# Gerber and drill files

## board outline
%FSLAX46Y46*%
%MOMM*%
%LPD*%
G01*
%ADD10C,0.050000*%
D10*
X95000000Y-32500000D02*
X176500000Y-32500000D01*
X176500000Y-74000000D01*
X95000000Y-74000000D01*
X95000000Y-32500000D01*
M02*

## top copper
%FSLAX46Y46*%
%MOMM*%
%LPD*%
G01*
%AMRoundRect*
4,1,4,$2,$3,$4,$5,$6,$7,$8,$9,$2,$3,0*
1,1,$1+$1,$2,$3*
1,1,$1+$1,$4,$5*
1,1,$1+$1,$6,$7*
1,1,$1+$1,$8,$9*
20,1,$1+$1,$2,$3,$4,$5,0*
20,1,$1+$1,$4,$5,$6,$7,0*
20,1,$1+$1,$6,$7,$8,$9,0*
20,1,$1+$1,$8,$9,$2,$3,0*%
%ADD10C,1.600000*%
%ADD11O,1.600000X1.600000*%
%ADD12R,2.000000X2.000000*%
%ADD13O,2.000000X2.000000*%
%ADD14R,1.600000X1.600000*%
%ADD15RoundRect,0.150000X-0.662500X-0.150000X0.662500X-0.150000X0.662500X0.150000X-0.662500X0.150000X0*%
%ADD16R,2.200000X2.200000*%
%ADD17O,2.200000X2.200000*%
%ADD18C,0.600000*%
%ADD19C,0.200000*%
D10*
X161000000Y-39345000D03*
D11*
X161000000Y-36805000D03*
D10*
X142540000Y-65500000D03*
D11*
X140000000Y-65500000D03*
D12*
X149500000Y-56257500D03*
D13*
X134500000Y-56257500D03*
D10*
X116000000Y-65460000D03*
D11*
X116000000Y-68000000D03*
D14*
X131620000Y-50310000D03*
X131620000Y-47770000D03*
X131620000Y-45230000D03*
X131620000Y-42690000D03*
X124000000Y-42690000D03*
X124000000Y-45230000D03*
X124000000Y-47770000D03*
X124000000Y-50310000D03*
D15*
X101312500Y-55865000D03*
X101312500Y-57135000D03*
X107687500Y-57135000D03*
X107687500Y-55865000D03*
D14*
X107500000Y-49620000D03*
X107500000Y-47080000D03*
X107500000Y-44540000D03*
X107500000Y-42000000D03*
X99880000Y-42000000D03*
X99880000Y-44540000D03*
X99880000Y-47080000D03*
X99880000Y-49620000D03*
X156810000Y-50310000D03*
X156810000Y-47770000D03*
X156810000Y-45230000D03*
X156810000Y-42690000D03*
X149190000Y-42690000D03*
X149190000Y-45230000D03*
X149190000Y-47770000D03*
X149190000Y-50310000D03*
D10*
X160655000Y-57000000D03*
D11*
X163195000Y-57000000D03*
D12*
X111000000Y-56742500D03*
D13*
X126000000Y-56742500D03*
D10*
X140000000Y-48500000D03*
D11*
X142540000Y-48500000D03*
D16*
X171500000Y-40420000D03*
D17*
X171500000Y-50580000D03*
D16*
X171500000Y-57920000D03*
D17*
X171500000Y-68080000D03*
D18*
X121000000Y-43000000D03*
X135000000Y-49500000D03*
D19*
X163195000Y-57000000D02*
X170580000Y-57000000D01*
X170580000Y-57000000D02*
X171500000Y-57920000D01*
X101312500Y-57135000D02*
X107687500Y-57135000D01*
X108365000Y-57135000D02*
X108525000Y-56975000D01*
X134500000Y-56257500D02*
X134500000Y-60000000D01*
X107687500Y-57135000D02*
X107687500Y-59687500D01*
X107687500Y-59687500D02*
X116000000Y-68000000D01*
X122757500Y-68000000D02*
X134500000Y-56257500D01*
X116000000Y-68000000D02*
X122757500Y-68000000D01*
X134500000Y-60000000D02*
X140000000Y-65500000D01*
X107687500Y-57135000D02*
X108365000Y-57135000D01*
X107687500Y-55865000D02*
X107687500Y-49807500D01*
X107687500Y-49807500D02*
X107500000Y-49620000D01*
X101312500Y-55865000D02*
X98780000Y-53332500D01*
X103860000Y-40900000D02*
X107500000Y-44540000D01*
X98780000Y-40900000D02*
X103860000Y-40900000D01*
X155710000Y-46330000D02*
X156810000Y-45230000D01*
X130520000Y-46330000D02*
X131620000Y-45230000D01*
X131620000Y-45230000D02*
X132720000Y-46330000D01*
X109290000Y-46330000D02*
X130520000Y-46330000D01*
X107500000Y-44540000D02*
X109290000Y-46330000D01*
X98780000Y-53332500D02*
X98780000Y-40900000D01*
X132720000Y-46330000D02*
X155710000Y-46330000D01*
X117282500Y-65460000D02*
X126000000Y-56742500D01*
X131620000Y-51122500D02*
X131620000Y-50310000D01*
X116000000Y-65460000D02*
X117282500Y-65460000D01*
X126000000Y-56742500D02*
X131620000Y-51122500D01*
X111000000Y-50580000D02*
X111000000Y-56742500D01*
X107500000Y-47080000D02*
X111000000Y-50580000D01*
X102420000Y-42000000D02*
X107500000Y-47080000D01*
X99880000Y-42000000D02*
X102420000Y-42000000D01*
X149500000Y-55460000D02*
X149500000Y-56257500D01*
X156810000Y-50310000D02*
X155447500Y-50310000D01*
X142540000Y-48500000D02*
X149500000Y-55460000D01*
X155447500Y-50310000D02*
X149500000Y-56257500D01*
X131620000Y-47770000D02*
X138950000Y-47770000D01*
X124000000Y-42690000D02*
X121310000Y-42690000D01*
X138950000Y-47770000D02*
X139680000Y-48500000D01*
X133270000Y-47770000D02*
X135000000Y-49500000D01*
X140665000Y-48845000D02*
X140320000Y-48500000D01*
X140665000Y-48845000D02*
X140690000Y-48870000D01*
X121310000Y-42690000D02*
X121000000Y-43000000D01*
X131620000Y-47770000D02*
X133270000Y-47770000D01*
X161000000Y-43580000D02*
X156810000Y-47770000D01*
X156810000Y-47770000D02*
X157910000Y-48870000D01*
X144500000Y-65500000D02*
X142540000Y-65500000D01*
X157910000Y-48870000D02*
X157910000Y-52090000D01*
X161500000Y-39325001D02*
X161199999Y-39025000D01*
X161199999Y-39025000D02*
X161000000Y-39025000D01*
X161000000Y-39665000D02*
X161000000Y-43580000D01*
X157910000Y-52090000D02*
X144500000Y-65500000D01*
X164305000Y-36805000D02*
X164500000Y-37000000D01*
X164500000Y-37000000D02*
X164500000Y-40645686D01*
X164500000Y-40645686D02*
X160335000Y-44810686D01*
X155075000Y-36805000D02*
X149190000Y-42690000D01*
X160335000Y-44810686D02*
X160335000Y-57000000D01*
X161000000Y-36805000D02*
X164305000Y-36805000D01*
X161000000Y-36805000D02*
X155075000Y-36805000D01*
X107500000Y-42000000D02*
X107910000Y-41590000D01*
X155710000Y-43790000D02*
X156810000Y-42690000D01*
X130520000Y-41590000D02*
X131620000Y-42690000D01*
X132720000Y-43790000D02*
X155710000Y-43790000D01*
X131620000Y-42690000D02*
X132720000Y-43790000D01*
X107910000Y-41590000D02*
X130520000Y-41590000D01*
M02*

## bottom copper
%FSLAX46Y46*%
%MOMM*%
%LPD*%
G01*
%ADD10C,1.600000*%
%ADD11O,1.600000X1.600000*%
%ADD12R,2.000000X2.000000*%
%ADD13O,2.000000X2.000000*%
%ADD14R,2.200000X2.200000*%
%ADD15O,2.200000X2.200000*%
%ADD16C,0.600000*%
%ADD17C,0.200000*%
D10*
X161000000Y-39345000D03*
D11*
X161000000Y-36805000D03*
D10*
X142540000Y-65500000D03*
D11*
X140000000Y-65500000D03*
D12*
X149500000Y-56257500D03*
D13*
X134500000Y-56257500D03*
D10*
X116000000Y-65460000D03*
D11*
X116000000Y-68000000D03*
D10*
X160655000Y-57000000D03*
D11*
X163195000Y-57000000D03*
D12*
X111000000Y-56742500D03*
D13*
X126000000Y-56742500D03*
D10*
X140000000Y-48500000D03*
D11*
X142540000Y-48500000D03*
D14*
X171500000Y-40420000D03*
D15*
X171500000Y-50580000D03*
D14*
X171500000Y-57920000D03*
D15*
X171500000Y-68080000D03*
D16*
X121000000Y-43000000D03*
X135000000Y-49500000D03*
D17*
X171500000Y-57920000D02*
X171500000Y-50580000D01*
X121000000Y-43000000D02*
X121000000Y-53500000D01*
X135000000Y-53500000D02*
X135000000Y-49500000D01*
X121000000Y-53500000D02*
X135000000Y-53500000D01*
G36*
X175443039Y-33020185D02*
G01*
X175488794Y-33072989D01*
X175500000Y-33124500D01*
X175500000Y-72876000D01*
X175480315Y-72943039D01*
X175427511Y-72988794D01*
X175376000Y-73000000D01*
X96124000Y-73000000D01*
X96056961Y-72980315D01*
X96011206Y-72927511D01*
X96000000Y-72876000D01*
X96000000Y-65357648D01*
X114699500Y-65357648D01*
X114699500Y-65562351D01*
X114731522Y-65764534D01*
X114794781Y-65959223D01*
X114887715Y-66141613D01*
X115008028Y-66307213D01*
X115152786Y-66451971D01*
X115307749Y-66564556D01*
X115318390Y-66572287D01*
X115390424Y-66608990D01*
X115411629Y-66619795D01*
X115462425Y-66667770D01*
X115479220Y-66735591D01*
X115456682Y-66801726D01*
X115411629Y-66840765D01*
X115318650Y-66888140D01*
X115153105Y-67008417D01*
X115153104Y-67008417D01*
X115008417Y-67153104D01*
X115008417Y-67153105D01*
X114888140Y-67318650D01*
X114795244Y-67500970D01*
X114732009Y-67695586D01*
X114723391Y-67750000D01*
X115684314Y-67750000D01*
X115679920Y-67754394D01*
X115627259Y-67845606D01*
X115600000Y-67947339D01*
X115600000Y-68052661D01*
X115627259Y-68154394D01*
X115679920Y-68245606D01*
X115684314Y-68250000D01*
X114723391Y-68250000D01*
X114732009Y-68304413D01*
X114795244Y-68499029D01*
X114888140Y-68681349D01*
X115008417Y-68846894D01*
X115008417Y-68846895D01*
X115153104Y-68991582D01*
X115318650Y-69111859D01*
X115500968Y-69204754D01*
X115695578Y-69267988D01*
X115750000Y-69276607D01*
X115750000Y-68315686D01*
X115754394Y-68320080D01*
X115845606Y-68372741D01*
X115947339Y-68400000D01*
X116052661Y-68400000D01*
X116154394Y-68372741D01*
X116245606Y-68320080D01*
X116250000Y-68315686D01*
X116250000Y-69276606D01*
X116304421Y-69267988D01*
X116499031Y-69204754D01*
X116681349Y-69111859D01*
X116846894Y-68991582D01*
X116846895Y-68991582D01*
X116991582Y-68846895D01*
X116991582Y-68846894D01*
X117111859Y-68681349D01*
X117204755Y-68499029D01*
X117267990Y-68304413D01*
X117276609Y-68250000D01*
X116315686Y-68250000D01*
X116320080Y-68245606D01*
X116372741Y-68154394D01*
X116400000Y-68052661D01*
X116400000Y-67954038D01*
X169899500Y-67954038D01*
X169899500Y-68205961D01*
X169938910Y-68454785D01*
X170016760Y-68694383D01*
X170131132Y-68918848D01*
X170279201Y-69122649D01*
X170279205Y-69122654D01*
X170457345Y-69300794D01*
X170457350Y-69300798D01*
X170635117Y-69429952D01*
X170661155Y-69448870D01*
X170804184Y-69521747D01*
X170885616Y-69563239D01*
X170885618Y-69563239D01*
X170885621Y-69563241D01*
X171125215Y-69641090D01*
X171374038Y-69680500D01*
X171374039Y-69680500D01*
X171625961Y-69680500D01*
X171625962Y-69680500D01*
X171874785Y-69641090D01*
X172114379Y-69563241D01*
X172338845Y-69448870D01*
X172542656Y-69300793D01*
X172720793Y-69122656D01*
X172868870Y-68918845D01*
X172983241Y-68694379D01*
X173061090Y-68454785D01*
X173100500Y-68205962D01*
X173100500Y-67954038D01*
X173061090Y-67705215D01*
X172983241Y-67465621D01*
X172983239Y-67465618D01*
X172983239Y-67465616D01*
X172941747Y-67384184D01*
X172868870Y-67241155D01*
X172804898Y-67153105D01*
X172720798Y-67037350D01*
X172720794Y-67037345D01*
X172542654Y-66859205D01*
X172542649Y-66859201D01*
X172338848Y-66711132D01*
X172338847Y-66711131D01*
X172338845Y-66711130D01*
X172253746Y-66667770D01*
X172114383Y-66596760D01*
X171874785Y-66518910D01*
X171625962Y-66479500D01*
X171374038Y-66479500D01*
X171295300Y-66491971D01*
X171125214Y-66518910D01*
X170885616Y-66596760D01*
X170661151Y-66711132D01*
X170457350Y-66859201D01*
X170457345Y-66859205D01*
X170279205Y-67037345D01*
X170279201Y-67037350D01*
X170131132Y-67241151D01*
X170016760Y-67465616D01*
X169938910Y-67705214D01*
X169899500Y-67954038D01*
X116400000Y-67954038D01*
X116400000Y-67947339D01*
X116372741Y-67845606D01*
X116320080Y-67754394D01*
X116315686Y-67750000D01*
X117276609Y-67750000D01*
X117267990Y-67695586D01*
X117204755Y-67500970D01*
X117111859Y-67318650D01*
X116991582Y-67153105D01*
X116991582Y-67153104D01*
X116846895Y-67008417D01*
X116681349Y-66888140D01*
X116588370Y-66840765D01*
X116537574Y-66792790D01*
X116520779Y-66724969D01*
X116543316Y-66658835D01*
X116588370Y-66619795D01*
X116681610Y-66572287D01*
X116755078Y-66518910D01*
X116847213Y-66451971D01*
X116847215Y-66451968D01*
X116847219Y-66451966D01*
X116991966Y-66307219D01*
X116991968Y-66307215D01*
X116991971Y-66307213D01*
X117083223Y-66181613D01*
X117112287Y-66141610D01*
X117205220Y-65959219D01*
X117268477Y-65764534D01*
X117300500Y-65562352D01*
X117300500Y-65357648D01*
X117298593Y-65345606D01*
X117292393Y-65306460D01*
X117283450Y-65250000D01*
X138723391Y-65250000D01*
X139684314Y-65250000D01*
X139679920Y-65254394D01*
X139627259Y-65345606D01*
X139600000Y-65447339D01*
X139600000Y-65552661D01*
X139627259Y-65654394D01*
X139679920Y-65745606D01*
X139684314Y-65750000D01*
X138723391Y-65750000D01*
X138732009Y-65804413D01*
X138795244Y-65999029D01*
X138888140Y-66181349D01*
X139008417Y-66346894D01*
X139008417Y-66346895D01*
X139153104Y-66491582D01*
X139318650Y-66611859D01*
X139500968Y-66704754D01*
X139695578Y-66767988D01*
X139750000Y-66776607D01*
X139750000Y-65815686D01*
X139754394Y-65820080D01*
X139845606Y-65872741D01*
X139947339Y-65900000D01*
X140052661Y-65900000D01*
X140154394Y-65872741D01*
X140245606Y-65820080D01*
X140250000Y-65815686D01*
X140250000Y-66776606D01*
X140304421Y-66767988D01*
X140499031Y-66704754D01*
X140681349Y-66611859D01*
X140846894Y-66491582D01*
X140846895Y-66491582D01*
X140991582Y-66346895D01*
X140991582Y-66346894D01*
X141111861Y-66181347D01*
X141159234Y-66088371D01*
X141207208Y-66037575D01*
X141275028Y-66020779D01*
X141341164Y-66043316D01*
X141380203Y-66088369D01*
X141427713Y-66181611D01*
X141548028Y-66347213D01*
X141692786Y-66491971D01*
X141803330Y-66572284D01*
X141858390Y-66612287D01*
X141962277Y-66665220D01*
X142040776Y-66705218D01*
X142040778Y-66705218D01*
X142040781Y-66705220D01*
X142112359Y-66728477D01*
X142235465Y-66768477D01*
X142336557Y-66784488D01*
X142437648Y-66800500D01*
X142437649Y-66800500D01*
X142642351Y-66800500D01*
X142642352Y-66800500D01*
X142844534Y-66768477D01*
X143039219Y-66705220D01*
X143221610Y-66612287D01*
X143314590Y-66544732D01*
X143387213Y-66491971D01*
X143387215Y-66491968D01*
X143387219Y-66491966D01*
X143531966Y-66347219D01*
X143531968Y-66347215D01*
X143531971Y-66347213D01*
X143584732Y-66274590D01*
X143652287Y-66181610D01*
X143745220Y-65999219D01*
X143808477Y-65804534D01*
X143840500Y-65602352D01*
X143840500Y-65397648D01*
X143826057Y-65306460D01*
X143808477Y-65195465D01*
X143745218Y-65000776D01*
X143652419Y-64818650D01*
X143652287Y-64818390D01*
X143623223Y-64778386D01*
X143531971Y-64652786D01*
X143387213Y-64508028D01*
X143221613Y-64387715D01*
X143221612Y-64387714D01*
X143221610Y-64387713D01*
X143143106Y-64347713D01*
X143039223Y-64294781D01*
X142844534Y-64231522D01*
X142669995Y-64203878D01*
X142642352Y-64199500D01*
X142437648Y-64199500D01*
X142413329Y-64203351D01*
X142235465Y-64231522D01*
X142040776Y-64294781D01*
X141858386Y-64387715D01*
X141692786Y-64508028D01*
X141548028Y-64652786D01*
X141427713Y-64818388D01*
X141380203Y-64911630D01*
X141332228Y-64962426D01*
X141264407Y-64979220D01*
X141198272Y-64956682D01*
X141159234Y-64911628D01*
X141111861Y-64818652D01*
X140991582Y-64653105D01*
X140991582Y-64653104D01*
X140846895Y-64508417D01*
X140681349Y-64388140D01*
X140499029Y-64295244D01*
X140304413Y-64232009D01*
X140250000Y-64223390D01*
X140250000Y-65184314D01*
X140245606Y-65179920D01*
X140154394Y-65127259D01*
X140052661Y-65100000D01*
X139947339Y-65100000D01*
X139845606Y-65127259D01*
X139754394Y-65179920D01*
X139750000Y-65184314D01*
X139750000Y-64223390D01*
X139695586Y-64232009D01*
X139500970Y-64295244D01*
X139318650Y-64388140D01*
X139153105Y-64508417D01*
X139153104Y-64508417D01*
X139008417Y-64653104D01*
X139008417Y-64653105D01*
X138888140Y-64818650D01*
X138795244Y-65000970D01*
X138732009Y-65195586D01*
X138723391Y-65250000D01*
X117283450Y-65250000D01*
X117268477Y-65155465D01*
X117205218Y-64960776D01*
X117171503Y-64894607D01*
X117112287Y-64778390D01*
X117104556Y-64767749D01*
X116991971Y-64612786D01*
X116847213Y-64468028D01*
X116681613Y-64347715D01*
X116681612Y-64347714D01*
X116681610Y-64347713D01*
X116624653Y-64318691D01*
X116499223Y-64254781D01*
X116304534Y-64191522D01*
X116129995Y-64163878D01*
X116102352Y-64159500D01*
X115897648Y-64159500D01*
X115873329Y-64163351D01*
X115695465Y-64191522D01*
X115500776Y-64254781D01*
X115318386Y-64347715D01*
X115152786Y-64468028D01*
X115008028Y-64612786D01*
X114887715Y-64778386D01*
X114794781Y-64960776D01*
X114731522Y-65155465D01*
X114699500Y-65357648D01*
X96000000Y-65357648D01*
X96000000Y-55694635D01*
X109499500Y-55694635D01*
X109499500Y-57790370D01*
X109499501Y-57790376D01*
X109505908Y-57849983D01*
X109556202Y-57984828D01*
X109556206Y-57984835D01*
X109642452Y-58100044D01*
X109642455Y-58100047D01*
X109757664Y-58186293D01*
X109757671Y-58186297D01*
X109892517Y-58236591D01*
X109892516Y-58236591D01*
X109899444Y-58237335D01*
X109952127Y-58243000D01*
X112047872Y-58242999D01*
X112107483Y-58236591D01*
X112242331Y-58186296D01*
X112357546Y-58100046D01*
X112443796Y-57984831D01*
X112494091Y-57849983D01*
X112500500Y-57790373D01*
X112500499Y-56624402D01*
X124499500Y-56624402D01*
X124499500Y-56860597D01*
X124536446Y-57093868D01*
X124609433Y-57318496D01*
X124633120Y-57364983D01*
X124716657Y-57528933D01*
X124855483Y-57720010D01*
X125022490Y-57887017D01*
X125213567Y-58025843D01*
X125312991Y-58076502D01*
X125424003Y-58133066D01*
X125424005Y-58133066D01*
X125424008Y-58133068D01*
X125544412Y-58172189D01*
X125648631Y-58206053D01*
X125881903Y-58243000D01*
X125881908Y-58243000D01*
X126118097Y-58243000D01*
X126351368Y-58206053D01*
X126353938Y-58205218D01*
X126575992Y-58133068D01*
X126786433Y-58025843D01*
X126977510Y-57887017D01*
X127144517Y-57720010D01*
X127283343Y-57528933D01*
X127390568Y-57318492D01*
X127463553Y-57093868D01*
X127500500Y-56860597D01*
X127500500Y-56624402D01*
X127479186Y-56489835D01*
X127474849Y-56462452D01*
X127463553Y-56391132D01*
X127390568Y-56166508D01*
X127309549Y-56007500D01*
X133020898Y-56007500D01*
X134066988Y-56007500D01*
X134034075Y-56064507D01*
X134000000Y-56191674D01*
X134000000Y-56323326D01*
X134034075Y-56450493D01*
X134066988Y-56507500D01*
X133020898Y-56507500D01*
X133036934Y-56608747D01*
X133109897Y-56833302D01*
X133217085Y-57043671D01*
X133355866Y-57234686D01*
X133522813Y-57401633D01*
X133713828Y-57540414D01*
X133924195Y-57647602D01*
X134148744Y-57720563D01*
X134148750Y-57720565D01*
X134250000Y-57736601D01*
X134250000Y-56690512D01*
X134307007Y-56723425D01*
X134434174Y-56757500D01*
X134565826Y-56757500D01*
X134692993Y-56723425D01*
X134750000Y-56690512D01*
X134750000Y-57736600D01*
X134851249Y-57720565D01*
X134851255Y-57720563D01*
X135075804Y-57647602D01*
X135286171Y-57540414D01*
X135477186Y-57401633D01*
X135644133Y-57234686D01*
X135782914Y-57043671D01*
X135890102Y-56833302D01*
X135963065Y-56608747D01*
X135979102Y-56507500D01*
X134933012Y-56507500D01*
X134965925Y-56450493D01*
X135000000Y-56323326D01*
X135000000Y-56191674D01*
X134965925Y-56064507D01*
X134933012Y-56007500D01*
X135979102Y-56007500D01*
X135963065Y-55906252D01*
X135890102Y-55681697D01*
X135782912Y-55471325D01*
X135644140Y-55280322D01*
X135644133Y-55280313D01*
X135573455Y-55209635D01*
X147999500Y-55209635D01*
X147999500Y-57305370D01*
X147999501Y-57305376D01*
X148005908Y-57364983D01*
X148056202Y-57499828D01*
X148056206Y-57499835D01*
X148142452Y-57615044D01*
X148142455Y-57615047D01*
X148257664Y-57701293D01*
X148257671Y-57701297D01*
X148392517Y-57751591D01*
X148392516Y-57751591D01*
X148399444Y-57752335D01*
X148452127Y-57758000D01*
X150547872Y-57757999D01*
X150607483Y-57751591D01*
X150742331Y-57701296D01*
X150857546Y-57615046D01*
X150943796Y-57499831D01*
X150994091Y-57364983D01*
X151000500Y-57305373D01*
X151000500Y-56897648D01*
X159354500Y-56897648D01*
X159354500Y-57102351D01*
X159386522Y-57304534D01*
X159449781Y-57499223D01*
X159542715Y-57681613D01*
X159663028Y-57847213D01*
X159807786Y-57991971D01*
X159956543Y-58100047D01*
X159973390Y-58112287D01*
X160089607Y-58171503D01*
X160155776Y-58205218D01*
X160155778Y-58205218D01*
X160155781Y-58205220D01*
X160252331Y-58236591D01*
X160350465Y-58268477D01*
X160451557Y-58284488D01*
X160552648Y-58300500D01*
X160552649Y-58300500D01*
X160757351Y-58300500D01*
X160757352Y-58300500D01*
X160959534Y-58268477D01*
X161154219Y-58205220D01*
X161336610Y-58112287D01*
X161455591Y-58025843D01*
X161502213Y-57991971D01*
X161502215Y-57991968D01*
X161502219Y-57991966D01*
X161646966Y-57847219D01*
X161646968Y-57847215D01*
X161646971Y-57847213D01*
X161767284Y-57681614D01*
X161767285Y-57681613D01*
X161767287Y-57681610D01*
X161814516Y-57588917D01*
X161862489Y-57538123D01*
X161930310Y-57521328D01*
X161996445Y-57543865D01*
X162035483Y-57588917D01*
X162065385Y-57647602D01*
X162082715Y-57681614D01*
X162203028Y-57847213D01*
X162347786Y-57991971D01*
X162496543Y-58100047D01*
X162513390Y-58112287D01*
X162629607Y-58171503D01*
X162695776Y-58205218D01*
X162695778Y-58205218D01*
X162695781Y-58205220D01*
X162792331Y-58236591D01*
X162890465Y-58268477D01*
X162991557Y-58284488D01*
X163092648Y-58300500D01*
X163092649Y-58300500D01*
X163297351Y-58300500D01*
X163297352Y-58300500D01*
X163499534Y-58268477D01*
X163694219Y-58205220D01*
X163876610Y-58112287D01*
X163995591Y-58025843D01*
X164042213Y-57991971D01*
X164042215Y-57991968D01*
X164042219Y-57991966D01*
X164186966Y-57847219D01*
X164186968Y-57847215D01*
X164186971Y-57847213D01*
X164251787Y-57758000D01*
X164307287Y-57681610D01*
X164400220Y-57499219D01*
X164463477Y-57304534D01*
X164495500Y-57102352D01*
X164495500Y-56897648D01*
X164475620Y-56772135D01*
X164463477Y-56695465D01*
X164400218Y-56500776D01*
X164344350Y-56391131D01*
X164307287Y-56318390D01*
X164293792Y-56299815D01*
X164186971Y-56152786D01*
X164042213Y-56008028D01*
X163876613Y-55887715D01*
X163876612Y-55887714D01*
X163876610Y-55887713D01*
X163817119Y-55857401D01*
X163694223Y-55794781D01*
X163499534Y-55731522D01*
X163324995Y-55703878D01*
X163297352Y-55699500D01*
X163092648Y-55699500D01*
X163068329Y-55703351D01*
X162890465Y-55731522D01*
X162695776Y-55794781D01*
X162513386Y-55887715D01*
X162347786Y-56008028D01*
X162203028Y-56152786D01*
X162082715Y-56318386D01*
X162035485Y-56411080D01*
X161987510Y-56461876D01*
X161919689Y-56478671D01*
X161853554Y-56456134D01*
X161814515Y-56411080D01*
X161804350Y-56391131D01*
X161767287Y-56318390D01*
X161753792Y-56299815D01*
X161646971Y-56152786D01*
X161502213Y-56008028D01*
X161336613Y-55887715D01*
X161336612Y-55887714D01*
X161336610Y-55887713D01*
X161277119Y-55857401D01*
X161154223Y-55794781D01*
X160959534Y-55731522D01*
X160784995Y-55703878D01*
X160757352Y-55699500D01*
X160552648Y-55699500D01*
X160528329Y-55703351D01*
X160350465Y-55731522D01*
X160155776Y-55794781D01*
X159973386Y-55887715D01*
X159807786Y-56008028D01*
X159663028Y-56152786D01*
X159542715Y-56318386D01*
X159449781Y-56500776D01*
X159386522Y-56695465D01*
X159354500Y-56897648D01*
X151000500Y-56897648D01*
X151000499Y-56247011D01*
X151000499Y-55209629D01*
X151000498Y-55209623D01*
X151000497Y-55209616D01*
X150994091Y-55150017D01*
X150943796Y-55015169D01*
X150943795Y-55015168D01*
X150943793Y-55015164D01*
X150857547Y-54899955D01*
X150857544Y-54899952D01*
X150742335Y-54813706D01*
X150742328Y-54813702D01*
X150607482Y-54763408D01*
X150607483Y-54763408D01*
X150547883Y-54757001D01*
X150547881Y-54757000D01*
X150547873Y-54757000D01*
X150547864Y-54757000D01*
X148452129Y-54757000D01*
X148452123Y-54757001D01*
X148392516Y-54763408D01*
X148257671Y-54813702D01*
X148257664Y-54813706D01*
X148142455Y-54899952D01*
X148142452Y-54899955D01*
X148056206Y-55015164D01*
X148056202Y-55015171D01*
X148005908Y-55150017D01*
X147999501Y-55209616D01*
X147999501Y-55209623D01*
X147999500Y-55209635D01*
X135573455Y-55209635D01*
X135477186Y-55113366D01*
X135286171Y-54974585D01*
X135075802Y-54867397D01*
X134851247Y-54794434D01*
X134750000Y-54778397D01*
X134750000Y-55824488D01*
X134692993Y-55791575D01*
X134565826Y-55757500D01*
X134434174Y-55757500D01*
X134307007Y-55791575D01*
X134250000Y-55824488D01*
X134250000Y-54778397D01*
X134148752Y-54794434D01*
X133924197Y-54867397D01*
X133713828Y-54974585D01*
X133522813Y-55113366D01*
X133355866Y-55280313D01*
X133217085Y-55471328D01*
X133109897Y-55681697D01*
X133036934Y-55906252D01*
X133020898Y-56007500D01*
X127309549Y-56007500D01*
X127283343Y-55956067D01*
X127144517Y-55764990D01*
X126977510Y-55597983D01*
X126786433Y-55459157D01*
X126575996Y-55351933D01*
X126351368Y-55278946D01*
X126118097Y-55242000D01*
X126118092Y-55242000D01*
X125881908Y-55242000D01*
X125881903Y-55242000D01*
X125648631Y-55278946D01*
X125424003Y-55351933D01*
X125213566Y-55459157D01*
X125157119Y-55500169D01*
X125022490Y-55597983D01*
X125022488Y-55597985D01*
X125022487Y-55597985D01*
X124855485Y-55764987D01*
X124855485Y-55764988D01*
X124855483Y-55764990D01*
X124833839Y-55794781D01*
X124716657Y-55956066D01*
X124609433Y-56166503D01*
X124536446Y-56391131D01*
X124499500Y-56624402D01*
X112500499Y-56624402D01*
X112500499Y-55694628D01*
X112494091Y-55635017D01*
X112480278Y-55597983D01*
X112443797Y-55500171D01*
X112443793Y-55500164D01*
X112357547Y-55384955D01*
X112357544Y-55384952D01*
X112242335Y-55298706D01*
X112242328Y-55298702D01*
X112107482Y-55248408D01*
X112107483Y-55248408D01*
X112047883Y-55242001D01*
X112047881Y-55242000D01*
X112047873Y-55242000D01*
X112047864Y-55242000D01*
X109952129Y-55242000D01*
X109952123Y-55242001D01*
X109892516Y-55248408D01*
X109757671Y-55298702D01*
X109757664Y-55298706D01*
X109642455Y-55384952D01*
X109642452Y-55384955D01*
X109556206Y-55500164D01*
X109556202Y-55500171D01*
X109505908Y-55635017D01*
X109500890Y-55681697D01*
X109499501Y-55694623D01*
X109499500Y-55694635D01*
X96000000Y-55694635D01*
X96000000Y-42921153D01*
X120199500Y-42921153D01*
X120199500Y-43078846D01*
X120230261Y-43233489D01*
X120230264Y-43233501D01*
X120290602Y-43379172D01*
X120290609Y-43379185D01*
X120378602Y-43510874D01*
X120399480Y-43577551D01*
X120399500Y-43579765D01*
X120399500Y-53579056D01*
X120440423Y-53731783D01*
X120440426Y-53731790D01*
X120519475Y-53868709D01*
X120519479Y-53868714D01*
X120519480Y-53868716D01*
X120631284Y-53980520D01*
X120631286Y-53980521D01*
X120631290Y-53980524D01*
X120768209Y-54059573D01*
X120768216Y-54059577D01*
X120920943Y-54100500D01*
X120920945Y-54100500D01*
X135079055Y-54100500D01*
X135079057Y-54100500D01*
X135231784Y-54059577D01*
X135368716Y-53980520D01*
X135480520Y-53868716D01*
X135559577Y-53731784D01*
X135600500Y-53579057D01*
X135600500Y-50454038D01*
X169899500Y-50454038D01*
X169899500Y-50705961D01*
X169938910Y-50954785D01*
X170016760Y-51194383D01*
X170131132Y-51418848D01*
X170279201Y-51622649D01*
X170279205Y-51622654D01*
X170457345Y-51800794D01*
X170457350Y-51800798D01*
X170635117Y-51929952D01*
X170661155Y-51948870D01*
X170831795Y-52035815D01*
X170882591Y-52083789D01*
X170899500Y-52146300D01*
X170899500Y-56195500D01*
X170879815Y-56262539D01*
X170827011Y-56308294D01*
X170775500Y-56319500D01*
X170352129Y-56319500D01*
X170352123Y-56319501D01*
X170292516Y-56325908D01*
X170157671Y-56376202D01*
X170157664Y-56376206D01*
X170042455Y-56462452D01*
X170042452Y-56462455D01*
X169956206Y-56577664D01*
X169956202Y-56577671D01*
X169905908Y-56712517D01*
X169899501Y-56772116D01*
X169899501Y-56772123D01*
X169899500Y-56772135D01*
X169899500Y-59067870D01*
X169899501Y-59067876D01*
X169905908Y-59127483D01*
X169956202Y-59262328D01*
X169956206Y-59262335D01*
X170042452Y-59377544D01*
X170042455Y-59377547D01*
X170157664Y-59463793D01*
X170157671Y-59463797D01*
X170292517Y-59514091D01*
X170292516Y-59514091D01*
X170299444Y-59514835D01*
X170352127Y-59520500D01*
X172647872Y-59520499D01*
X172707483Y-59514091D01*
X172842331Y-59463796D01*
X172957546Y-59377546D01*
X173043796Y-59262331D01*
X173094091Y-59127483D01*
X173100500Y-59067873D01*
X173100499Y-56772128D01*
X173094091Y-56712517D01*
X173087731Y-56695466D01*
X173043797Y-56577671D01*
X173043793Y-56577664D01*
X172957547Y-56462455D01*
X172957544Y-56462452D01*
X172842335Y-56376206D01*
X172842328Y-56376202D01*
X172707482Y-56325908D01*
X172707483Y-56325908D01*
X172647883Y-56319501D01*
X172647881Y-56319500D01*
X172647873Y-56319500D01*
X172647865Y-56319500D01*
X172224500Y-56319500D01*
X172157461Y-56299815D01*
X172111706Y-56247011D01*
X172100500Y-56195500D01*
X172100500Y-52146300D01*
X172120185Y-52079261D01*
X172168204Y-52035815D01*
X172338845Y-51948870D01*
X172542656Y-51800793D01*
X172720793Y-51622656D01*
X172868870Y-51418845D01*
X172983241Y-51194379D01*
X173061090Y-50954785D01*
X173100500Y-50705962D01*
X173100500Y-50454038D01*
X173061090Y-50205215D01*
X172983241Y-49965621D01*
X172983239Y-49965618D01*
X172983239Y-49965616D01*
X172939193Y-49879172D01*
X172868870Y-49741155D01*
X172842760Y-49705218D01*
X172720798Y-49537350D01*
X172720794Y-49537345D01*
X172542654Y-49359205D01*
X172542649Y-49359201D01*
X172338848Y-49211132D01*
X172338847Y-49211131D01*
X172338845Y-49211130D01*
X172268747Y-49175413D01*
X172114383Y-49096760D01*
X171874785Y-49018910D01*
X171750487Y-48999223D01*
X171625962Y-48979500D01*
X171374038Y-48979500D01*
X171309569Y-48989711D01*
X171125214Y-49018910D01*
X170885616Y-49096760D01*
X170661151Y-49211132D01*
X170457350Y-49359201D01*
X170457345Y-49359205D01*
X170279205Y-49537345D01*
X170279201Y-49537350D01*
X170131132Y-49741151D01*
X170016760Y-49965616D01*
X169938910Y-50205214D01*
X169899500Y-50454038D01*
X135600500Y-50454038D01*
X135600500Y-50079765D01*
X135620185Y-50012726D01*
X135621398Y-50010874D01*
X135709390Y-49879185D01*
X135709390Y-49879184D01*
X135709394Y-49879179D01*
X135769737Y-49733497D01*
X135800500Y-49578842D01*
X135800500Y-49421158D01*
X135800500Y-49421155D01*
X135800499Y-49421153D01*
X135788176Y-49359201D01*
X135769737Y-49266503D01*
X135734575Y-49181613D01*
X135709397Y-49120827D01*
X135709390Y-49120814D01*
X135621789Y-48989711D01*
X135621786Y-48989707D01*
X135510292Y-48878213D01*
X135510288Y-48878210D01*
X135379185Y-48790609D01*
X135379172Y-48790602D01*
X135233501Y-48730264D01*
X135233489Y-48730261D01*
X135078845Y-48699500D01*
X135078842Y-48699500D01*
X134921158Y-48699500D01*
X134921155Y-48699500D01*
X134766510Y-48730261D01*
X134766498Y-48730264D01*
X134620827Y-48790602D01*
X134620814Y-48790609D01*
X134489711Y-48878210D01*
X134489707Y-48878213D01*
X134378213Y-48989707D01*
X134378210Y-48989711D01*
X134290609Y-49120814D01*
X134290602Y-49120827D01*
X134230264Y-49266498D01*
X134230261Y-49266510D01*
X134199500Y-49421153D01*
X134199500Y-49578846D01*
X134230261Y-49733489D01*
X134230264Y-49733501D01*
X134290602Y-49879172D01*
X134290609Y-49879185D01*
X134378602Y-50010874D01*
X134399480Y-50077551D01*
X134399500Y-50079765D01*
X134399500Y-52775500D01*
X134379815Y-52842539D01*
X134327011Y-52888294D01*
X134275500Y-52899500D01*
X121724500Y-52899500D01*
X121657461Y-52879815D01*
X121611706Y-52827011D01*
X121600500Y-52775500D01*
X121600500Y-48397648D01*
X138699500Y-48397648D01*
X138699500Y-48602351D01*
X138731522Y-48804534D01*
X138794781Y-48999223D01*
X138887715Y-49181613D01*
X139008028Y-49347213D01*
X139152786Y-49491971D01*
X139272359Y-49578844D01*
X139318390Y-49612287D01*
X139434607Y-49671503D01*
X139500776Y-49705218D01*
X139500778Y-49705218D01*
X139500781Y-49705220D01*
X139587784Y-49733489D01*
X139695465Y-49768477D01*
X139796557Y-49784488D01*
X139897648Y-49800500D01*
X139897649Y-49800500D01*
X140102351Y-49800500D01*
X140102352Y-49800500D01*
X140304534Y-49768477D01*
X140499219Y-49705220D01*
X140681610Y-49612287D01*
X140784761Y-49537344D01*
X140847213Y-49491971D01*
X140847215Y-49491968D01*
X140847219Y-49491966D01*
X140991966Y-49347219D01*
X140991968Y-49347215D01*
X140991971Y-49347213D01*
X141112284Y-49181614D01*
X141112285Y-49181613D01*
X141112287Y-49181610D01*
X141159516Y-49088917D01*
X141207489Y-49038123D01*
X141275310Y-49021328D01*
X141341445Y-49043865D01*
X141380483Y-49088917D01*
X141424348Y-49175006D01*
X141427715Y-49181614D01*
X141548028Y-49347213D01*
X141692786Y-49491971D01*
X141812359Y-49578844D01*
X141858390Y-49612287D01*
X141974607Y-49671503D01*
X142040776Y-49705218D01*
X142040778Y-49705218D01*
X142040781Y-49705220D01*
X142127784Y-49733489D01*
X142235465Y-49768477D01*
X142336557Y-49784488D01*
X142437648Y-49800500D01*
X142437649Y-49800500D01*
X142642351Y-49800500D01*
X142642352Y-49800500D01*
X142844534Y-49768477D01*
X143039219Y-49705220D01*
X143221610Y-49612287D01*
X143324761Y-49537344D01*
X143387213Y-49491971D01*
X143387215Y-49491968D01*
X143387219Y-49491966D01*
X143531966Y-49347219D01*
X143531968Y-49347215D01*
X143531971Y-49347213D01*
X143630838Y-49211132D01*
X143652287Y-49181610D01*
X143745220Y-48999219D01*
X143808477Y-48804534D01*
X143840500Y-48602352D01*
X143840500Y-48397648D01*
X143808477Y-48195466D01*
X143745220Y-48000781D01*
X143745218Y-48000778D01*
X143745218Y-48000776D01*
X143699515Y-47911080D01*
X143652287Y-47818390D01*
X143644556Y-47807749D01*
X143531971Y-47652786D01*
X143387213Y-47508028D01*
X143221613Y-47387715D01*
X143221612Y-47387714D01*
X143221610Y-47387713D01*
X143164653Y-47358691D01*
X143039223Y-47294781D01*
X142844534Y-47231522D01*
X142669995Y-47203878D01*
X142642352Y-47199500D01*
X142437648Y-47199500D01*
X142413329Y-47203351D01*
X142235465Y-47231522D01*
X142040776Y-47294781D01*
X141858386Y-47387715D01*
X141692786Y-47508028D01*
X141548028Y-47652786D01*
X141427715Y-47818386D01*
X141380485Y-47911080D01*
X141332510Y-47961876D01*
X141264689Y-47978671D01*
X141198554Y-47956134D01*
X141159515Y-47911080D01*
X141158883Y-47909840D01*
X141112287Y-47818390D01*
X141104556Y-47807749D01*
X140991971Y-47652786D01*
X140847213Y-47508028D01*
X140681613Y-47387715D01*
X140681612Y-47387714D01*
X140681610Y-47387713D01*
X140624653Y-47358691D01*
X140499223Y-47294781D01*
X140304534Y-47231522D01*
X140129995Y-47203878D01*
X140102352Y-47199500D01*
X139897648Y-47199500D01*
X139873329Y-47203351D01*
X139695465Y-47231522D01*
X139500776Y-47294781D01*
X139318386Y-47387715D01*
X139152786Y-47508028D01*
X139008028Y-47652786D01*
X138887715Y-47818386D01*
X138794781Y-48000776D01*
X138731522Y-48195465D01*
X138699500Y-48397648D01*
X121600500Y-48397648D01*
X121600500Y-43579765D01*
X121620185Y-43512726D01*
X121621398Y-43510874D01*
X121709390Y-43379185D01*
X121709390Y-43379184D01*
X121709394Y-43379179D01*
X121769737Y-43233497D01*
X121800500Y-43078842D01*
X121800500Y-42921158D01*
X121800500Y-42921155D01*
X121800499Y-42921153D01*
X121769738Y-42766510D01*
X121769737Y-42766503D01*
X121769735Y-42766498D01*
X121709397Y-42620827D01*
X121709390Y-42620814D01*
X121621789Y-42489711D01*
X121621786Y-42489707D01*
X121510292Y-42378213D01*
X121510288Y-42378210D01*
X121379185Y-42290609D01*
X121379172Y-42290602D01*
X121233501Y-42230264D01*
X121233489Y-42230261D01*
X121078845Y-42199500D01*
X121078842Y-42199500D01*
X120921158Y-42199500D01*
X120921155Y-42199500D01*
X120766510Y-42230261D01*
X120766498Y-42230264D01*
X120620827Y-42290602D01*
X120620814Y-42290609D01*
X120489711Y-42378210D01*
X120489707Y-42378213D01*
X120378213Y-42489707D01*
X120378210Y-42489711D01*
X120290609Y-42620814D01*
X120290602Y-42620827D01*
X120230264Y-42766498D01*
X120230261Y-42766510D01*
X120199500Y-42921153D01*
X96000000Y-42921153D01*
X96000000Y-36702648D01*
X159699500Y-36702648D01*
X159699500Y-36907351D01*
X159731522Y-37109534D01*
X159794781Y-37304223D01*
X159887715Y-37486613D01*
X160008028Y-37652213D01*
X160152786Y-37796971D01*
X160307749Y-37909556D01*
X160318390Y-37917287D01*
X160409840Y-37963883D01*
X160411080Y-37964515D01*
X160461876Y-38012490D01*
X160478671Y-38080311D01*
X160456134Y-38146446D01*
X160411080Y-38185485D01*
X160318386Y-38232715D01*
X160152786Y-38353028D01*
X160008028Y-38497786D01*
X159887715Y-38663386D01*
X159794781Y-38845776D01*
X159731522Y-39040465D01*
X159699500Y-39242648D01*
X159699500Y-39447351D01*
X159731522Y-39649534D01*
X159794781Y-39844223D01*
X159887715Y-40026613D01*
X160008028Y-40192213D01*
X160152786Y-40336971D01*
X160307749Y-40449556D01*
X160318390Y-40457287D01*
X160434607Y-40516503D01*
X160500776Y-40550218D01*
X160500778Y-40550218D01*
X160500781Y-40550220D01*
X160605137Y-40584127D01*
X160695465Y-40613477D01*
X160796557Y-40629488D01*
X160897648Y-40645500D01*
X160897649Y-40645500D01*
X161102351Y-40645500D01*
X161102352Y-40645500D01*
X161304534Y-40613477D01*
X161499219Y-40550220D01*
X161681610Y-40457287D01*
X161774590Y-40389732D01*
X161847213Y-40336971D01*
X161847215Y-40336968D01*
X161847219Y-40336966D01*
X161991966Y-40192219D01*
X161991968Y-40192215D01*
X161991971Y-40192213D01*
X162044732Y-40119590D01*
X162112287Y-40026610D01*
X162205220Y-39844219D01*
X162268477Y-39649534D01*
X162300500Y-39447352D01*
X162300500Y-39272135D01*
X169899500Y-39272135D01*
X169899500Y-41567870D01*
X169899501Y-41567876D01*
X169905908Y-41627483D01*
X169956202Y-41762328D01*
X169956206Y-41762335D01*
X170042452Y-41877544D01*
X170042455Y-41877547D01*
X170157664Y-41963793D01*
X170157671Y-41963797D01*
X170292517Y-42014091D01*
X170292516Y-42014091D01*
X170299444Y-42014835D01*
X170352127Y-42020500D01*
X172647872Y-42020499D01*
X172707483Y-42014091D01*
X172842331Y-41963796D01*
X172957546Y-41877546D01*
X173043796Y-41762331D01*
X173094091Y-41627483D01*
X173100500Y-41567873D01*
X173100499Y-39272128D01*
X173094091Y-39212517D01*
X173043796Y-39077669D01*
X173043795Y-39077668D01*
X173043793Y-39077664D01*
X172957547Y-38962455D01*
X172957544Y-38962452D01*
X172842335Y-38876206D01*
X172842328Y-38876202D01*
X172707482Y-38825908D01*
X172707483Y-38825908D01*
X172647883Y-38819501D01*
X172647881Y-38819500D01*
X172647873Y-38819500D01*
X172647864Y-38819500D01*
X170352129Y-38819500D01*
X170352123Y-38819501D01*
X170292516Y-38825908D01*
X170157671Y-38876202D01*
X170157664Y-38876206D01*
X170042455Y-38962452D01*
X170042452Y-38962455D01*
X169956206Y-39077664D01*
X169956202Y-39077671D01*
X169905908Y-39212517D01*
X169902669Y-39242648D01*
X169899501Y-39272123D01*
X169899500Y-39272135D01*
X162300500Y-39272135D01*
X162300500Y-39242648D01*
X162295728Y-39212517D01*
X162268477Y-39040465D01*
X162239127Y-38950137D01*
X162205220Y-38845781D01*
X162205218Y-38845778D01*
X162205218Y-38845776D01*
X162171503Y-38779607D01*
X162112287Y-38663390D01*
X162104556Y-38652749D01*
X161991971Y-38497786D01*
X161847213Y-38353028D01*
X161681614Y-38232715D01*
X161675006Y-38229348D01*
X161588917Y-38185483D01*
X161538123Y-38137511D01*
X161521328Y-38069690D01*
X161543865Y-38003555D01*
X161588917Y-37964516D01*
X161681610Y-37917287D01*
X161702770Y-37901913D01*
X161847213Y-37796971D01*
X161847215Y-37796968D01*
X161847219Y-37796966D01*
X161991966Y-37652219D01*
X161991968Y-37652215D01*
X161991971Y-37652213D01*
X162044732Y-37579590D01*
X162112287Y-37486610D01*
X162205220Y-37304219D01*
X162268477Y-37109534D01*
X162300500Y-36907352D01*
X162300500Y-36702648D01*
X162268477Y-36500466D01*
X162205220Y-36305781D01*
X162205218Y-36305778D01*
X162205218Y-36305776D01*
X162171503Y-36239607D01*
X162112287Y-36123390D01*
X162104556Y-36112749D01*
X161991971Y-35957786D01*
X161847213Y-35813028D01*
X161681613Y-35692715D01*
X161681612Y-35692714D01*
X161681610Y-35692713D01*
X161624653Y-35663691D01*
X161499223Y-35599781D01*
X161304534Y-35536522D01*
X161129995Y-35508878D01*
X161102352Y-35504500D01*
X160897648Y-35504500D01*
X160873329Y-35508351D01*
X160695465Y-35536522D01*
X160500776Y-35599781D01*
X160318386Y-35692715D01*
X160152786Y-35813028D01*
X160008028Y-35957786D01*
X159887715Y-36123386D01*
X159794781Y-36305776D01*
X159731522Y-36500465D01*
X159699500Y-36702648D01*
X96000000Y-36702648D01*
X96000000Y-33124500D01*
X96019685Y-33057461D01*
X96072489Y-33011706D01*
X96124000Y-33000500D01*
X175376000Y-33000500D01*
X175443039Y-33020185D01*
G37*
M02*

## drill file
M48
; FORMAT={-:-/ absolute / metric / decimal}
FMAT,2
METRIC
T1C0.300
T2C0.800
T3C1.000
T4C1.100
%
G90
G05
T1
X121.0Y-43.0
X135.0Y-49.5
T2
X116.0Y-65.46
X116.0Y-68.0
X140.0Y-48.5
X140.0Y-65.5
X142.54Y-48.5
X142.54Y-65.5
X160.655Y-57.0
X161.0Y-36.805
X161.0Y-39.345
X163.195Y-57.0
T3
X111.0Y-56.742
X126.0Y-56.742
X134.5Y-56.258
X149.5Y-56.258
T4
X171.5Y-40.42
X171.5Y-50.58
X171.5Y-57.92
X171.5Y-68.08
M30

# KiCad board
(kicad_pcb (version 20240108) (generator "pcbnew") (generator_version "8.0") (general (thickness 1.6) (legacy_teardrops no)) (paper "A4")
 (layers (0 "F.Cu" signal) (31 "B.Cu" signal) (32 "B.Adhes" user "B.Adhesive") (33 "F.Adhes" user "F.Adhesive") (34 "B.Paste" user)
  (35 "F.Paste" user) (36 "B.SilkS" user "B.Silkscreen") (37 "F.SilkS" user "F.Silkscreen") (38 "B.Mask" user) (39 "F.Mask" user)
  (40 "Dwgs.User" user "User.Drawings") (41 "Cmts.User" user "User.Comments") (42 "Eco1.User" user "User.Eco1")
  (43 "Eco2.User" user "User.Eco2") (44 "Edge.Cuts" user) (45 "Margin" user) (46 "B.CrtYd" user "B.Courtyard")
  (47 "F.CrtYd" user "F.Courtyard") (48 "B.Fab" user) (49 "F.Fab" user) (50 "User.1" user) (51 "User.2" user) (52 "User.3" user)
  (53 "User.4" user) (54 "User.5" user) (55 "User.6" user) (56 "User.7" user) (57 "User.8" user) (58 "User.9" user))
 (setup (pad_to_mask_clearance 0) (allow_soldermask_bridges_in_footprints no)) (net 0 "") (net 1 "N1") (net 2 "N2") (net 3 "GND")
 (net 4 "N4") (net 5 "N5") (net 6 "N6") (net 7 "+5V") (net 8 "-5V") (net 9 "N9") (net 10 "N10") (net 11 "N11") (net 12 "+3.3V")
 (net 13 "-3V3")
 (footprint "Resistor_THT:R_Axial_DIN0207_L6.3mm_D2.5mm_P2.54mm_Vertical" (layer "F.Cu") (at 161 39.345 90)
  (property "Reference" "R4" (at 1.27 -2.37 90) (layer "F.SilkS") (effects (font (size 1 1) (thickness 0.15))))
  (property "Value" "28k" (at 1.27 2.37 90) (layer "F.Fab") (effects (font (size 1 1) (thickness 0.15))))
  (pad "1" thru_hole circle (at 0 0 90) (size 1.6 1.6) (drill 0.8) (layers "*.Cu" "*.Mask") (remove_unused_layers no) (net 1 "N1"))
  (pad "2" thru_hole oval (at 2.54 0 90) (size 1.6 1.6) (drill 0.8) (layers "*.Cu" "*.Mask") (remove_unused_layers no) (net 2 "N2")))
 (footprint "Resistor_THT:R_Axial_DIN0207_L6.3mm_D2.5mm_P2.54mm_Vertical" (layer "F.Cu") (at 142.54 65.5 180)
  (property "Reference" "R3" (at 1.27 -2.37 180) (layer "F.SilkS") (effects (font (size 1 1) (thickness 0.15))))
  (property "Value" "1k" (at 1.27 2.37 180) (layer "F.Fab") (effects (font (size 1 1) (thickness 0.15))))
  (pad "1" thru_hole circle (at 0 0 180) (size 1.6 1.6) (drill 0.8) (layers "*.Cu" "*.Mask") (remove_unused_layers no) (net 1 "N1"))
  (pad "2" thru_hole oval (at 2.54 0 180) (size 1.6 1.6) (drill 0.8) (layers "*.Cu" "*.Mask") (remove_unused_layers no) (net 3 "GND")))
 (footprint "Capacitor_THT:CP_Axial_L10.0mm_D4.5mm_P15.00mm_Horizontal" (layer "F.Cu") (at 149.5 56.2575 180)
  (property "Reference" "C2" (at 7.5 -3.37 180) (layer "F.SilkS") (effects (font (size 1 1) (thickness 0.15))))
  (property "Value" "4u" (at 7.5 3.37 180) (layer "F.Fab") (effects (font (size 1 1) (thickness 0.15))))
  (pad "1" thru_hole rect (at 0 0 180) (size 2 2) (drill 1) (layers "*.Cu" "*.Mask") (remove_unused_layers no) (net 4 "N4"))
  (pad "2" thru_hole oval (at 15 0 180) (size 2 2) (drill 1) (layers "*.Cu" "*.Mask") (remove_unused_layers no) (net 3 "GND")))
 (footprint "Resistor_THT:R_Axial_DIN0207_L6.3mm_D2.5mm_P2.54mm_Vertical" (layer "F.Cu") (at 116 65.46 -90)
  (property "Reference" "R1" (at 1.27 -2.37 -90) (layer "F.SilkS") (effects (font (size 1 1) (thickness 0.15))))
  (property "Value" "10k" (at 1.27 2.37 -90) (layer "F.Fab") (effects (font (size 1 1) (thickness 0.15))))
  (pad "1" thru_hole circle (at 0 0 270) (size 1.6 1.6) (drill 0.8) (layers "*.Cu" "*.Mask") (remove_unused_layers no) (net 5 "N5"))
  (pad "2" thru_hole oval (at 2.54 0 270) (size 1.6 1.6) (drill 0.8) (layers "*.Cu" "*.Mask") (remove_unused_layers no) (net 3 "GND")))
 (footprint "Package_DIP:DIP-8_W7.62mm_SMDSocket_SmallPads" (layer "F.Cu") (at 127.81 46.5 180)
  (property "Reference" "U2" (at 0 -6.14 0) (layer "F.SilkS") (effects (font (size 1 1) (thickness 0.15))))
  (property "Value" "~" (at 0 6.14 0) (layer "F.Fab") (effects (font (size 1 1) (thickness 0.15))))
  (pad "1" smd rect (at -3.81 -3.81 180) (size 1.6 1.6) (layers "F.Cu" "F.Paste" "F.Mask") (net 5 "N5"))
  (pad "2" smd rect (at -3.81 -1.27 180) (size 1.6 1.6) (layers "F.Cu" "F.Paste" "F.Mask") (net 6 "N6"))
  (pad "3" smd rect (at -3.81 1.27 180) (size 1.6 1.6) (layers "F.Cu" "F.Paste" "F.Mask") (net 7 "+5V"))
  (pad "4" smd rect (at -3.81 3.81 180) (size 1.6 1.6) (layers "F.Cu" "F.Paste" "F.Mask") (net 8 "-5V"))
  (pad "5" smd rect (at 3.81 3.81 180) (size 1.6 1.6) (layers "F.Cu" "F.Paste" "F.Mask") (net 6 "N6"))
  (pad "6" smd rect (at 3.81 1.27 180) (size 1.6 1.6) (layers "F.Cu" "F.Paste" "F.Mask"))
  (pad "7" smd rect (at 3.81 -1.27 180) (size 1.6 1.6) (layers "F.Cu" "F.Paste" "F.Mask"))
  (pad "8" smd rect (at 3.81 -3.81 180) (size 1.6 1.6) (layers "F.Cu" "F.Paste" "F.Mask")))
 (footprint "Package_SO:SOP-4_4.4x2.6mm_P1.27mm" (layer "F.Cu") (at 104.5 56.5)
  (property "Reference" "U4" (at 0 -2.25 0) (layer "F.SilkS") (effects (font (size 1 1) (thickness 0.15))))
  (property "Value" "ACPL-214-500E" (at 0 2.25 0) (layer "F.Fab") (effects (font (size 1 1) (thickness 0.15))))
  (pad "1" smd roundrect (at -3.1875 -0.635) (size 1.625 0.6) (layers "F.Cu" "F.Paste" "F.Mask") (roundrect_rratio 0.25) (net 7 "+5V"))
  (pad "2" smd roundrect (at -3.1875 0.635) (size 1.625 0.6) (layers "F.Cu" "F.Paste" "F.Mask") (roundrect_rratio 0.25) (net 3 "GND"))
  (pad "3" smd roundrect (at 3.1875 0.635) (size 1.625 0.6) (layers "F.Cu" "F.Paste" "F.Mask") (roundrect_rratio 0.25) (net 3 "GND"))
  (pad "4" smd roundrect (at 3.1875 -0.635) (size 1.625 0.6) (layers "F.Cu" "F.Paste" "F.Mask") (roundrect_rratio 0.25) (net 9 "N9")))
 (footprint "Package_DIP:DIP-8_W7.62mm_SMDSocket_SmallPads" (layer "F.Cu") (at 103.69 45.81 180)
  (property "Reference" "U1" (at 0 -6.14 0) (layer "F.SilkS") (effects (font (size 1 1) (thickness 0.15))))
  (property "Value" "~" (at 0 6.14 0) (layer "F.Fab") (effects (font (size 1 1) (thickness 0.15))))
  (pad "1" smd rect (at -3.81 -3.81 180) (size 1.6 1.6) (layers "F.Cu" "F.Paste" "F.Mask") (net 9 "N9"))
  (pad "2" smd rect (at -3.81 -1.27 180) (size 1.6 1.6) (layers "F.Cu" "F.Paste" "F.Mask") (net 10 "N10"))
  (pad "3" smd rect (at -3.81 1.27 180) (size 1.6 1.6) (layers "F.Cu" "F.Paste" "F.Mask") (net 7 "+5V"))
  (pad "4" smd rect (at -3.81 3.81 180) (size 1.6 1.6) (layers "F.Cu" "F.Paste" "F.Mask") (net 8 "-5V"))
  (pad "5" smd rect (at 3.81 3.81 180) (size 1.6 1.6) (layers "F.Cu" "F.Paste" "F.Mask") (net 10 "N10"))
  (pad "6" smd rect (at 3.81 1.27 180) (size 1.6 1.6) (layers "F.Cu" "F.Paste" "F.Mask"))
  (pad "7" smd rect (at 3.81 -1.27 180) (size 1.6 1.6) (layers "F.Cu" "F.Paste" "F.Mask"))
  (pad "8" smd rect (at 3.81 -3.81 180) (size 1.6 1.6) (layers "F.Cu" "F.Paste" "F.Mask")))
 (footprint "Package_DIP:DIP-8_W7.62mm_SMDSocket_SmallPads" (layer "F.Cu") (at 153 46.5 180)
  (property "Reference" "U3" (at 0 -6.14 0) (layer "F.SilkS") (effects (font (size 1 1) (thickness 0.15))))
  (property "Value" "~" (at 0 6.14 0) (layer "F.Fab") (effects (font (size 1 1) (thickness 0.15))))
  (pad "1" smd rect (at -3.81 -3.81 180) (size 1.6 1.6) (layers "F.Cu" "F.Paste" "F.Mask") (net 4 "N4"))
  (pad "2" smd rect (at -3.81 -1.27 180) (size 1.6 1.6) (layers "F.Cu" "F.Paste" "F.Mask") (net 1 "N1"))
  (pad "3" smd rect (at -3.81 1.27 180) (size 1.6 1.6) (layers "F.Cu" "F.Paste" "F.Mask") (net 7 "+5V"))
  (pad "4" smd rect (at -3.81 3.81 180) (size 1.6 1.6) (layers "F.Cu" "F.Paste" "F.Mask") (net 8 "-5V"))
  (pad "5" smd rect (at 3.81 3.81 180) (size 1.6 1.6) (layers "F.Cu" "F.Paste" "F.Mask") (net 2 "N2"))
  (pad "6" smd rect (at 3.81 1.27 180) (size 1.6 1.6) (layers "F.Cu" "F.Paste" "F.Mask"))
  (pad "7" smd rect (at 3.81 -1.27 180) (size 1.6 1.6) (layers "F.Cu" "F.Paste" "F.Mask"))
  (pad "8" smd rect (at 3.81 -3.81 180) (size 1.6 1.6) (layers "F.Cu" "F.Paste" "F.Mask")))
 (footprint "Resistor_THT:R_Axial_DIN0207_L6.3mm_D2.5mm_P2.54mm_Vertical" (layer "F.Cu") (at 160.655 57)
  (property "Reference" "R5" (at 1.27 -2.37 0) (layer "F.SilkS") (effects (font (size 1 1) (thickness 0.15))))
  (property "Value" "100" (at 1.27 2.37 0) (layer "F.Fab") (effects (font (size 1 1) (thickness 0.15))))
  (pad "1" thru_hole circle (at 0 0) (size 1.6 1.6) (drill 0.8) (layers "*.Cu" "*.Mask") (remove_unused_layers no) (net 2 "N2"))
  (pad "2" thru_hole oval (at 2.54 0) (size 1.6 1.6) (drill 0.8) (layers "*.Cu" "*.Mask") (remove_unused_layers no) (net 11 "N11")))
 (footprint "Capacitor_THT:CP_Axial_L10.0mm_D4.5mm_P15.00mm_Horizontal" (layer "F.Cu") (at 111 56.7425)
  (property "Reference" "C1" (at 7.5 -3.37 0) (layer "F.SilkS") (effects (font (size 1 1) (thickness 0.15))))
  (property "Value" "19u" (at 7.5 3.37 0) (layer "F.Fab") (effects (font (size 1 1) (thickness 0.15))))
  (pad "1" thru_hole rect (at 0 0) (size 2 2) (drill 1) (layers "*.Cu" "*.Mask") (remove_unused_layers no) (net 10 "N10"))
  (pad "2" thru_hole oval (at 15 0) (size 2 2) (drill 1) (layers "*.Cu" "*.Mask") (remove_unused_layers no) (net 5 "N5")))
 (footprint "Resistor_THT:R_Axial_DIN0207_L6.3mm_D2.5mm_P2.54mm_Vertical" (layer "F.Cu") (at 140 48.5)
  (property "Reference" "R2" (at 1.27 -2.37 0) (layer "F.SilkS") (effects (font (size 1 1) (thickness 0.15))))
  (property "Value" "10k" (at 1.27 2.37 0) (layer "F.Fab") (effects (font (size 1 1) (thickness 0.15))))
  (pad "1" thru_hole circle (at 0 0) (size 1.6 1.6) (drill 0.8) (layers "*.Cu" "*.Mask") (remove_unused_layers no) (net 6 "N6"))
  (pad "2" thru_hole oval (at 2.54 0) (size 1.6 1.6) (drill 0.8) (layers "*.Cu" "*.Mask") (remove_unused_layers no) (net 4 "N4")))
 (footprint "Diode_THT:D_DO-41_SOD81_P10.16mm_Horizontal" (layer "F.Cu") (at 171.5 40.42 -90)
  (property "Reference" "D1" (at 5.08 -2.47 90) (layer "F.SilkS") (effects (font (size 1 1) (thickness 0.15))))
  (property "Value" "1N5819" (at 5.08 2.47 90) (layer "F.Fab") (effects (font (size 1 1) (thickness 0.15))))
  (pad "1" thru_hole rect (at 0 0 270) (size 2.2 2.2) (drill 1.1) (layers "*.Cu" "*.Mask") (remove_unused_layers no) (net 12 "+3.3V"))
  (pad "2" thru_hole oval (at 10.16 0 270) (size 2.2 2.2) (drill 1.1) (layers "*.Cu" "*.Mask") (remove_unused_layers no) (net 11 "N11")))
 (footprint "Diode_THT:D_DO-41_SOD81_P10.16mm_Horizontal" (layer "F.Cu") (at 171.5 57.92 -90)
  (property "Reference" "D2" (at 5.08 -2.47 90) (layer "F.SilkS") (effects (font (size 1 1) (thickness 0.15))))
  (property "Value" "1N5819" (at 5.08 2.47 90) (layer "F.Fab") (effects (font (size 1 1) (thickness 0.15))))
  (pad "1" thru_hole rect (at 0 0 270) (size 2.2 2.2) (drill 1.1) (layers "*.Cu" "*.Mask") (remove_unused_layers no) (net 11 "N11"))
  (pad "2" thru_hole oval (at 10.16 0 270) (size 2.2 2.2) (drill 1.1) (layers "*.Cu" "*.Mask") (remove_unused_layers no) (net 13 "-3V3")))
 (gr_poly (pts (xy 95 32.5) (xy 176.5 32.5) (xy 176.5 74) (xy 95 74)) (stroke (width 0.05) (type solid)) (fill none) (layer "Edge.Cuts"))
 (segment (start 163.195 57) (end 170.58 57) (width 0.2) (layer "F.Cu") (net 11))
 (segment (start 170.58 57) (end 171.5 57.92) (width 0.2) (layer "F.Cu") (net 11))
 (segment (start 171.5 57.92) (end 171.5 50.58) (width 0.2) (layer "B.Cu") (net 11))
 (segment (start 101.3125 57.135) (end 107.6875 57.135) (width 0.2) (layer "F.Cu") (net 3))
 (segment (start 108.365 57.135) (end 108.525 56.975) (width 0.2) (layer "F.Cu") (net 3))
 (segment (start 134.5 56.2575) (end 134.5 60) (width 0.2) (layer "F.Cu") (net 3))
 (segment (start 107.6875 57.135) (end 107.6875 59.6875) (width 0.2) (layer "F.Cu") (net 3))
 (segment (start 107.6875 59.6875) (end 116 68) (width 0.2) (layer "F.Cu") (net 3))
 (segment (start 122.7575 68) (end 134.5 56.2575) (width 0.2) (layer "F.Cu") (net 3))
 (segment (start 116 68) (end 122.7575 68) (width 0.2) (layer "F.Cu") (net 3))
 (segment (start 134.5 60) (end 140 65.5) (width 0.2) (layer "F.Cu") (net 3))
 (segment (start 107.6875 57.135) (end 108.365 57.135) (width 0.2) (layer "F.Cu") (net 3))
 (segment (start 107.6875 55.865) (end 107.6875 49.8075) (width 0.2) (layer "F.Cu") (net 9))
 (segment (start 107.6875 49.8075) (end 107.5 49.62) (width 0.2) (layer "F.Cu") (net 9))
 (segment (start 101.3125 55.865) (end 98.78 53.3325) (width 0.2) (layer "F.Cu") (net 7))
 (segment (start 103.86 40.9) (end 107.5 44.54) (width 0.2) (layer "F.Cu") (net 7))
 (segment (start 98.78 40.9) (end 103.86 40.9) (width 0.2) (layer "F.Cu") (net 7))
 (segment (start 155.71 46.33) (end 156.81 45.23) (width 0.2) (layer "F.Cu") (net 7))
 (segment (start 130.52 46.33) (end 131.62 45.23) (width 0.2) (layer "F.Cu") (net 7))
 (segment (start 131.62 45.23) (end 132.72 46.33) (width 0.2) (layer "F.Cu") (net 7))
 (segment (start 109.29 46.33) (end 130.52 46.33) (width 0.2) (layer "F.Cu") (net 7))
 (segment (start 107.5 44.54) (end 109.29 46.33) (width 0.2) (layer "F.Cu") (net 7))
 (segment (start 98.78 53.3325) (end 98.78 40.9) (width 0.2) (layer "F.Cu") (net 7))
 (segment (start 132.72 46.33) (end 155.71 46.33) (width 0.2) (layer "F.Cu") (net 7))
 (segment (start 117.2825 65.46) (end 126 56.7425) (width 0.2) (layer "F.Cu") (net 5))
 (segment (start 131.62 51.1225) (end 131.62 50.31) (width 0.2) (layer "F.Cu") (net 5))
 (segment (start 116 65.46) (end 117.2825 65.46) (width 0.2) (layer "F.Cu") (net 5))
 (segment (start 126 56.7425) (end 131.62 51.1225) (width 0.2) (layer "F.Cu") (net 5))
 (segment (start 111 50.58) (end 111 56.7425) (width 0.2) (layer "F.Cu") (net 10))
 (segment (start 107.5 47.08) (end 111 50.58) (width 0.2) (layer "F.Cu") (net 10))
 (segment (start 102.42 42) (end 107.5 47.08) (width 0.2) (layer "F.Cu") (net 10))
 (segment (start 99.88 42) (end 102.42 42) (width 0.2) (layer "F.Cu") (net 10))
 (segment (start 149.5 55.46) (end 149.5 56.2575) (width 0.2) (layer "F.Cu") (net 4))
 (segment (start 156.81 50.31) (end 155.4475 50.31) (width 0.2) (layer "F.Cu") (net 4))
 (segment (start 142.54 48.5) (end 149.5 55.46) (width 0.2) (layer "F.Cu") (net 4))
 (segment (start 155.4475 50.31) (end 149.5 56.2575) (width 0.2) (layer "F.Cu") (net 4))
 (segment (start 131.62 47.77) (end 138.95 47.77) (width 0.2) (layer "F.Cu") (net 6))
 (segment (start 124 42.69) (end 121.31 42.69) (width 0.2) (layer "F.Cu") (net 6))
 (segment (start 138.95 47.77) (end 139.68 48.5) (width 0.2) (layer "F.Cu") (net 6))
 (segment (start 133.27 47.77) (end 135 49.5) (width 0.2) (layer "F.Cu") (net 6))
 (segment (start 140.665 48.845) (end 140.32 48.5) (width 0.2) (layer "F.Cu") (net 6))
 (segment (start 140.665 48.845) (end 140.69 48.87) (width 0.2) (layer "F.Cu") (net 6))
 (segment (start 121.31 42.69) (end 121 43) (width 0.2) (layer "F.Cu") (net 6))
 (segment (start 131.62 47.77) (end 133.27 47.77) (width 0.2) (layer "F.Cu") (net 6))
 (via (at 121 43) (size 0.6) (drill 0.3) (layers "F.Cu" "B.Cu") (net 6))
 (via (at 135 49.5) (size 0.6) (drill 0.3) (layers "F.Cu" "B.Cu") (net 6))
 (segment (start 121 43) (end 121 53.5) (width 0.2) (layer "B.Cu") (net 6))
 (segment (start 135 53.5) (end 135 49.5) (width 0.2) (layer "B.Cu") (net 6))
 (segment (start 121 53.5) (end 135 53.5) (width 0.2) (layer "B.Cu") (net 6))
 (segment (start 161 43.58) (end 156.81 47.77) (width 0.2) (layer "F.Cu") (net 1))
 (segment (start 156.81 47.77) (end 157.91 48.87) (width 0.2) (layer "F.Cu") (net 1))
 (segment (start 144.5 65.5) (end 142.54 65.5) (width 0.2) (layer "F.Cu") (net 1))
 (segment (start 157.91 48.87) (end 157.91 52.09) (width 0.2) (layer "F.Cu") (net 1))
 (segment (start 161.5 39.325001) (end 161.199999 39.025) (width 0.2) (layer "F.Cu") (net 1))
 (segment (start 161.199999 39.025) (end 161 39.025) (width 0.2) (layer "F.Cu") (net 1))
 (segment (start 161 39.665) (end 161 43.58) (width 0.2) (layer "F.Cu") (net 1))
 (segment (start 157.91 52.09) (end 144.5 65.5) (width 0.2) (layer "F.Cu") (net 1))
 (segment (start 164.305 36.805) (end 164.5 37) (width 0.2) (layer "F.Cu") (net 2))
 (segment (start 164.5 37) (end 164.5 40.645686) (width 0.2) (layer "F.Cu") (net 2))
 (segment (start 164.5 40.645686) (end 160.335 44.810686) (width 0.2) (layer "F.Cu") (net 2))
 (segment (start 155.075 36.805) (end 149.19 42.69) (width 0.2) (layer "F.Cu") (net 2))
 (segment (start 160.335 44.810686) (end 160.335 57) (width 0.2) (layer "F.Cu") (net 2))
 (segment (start 161 36.805) (end 164.305 36.805) (width 0.2) (layer "F.Cu") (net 2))
 (segment (start 161 36.805) (end 155.075 36.805) (width 0.2) (layer "F.Cu") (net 2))
 (segment (start 107.5 42) (end 107.91 41.59) (width 0.2) (layer "F.Cu") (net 8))
 (segment (start 155.71 43.79) (end 156.81 42.69) (width 0.2) (layer "F.Cu") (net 8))
 (segment (start 130.52 41.59) (end 131.62 42.69) (width 0.2) (layer "F.Cu") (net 8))
 (segment (start 132.72 43.79) (end 155.71 43.79) (width 0.2) (layer "F.Cu") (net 8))
 (segment (start 131.62 42.69) (end 132.72 43.79) (width 0.2) (layer "F.Cu") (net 8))
 (segment (start 107.91 41.59) (end 130.52 41.59) (width 0.2) (layer "F.Cu") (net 8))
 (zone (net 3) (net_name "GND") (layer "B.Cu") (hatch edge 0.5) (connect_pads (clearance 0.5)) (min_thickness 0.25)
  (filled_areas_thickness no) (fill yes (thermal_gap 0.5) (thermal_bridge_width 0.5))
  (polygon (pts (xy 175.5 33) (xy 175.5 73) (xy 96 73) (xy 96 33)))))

